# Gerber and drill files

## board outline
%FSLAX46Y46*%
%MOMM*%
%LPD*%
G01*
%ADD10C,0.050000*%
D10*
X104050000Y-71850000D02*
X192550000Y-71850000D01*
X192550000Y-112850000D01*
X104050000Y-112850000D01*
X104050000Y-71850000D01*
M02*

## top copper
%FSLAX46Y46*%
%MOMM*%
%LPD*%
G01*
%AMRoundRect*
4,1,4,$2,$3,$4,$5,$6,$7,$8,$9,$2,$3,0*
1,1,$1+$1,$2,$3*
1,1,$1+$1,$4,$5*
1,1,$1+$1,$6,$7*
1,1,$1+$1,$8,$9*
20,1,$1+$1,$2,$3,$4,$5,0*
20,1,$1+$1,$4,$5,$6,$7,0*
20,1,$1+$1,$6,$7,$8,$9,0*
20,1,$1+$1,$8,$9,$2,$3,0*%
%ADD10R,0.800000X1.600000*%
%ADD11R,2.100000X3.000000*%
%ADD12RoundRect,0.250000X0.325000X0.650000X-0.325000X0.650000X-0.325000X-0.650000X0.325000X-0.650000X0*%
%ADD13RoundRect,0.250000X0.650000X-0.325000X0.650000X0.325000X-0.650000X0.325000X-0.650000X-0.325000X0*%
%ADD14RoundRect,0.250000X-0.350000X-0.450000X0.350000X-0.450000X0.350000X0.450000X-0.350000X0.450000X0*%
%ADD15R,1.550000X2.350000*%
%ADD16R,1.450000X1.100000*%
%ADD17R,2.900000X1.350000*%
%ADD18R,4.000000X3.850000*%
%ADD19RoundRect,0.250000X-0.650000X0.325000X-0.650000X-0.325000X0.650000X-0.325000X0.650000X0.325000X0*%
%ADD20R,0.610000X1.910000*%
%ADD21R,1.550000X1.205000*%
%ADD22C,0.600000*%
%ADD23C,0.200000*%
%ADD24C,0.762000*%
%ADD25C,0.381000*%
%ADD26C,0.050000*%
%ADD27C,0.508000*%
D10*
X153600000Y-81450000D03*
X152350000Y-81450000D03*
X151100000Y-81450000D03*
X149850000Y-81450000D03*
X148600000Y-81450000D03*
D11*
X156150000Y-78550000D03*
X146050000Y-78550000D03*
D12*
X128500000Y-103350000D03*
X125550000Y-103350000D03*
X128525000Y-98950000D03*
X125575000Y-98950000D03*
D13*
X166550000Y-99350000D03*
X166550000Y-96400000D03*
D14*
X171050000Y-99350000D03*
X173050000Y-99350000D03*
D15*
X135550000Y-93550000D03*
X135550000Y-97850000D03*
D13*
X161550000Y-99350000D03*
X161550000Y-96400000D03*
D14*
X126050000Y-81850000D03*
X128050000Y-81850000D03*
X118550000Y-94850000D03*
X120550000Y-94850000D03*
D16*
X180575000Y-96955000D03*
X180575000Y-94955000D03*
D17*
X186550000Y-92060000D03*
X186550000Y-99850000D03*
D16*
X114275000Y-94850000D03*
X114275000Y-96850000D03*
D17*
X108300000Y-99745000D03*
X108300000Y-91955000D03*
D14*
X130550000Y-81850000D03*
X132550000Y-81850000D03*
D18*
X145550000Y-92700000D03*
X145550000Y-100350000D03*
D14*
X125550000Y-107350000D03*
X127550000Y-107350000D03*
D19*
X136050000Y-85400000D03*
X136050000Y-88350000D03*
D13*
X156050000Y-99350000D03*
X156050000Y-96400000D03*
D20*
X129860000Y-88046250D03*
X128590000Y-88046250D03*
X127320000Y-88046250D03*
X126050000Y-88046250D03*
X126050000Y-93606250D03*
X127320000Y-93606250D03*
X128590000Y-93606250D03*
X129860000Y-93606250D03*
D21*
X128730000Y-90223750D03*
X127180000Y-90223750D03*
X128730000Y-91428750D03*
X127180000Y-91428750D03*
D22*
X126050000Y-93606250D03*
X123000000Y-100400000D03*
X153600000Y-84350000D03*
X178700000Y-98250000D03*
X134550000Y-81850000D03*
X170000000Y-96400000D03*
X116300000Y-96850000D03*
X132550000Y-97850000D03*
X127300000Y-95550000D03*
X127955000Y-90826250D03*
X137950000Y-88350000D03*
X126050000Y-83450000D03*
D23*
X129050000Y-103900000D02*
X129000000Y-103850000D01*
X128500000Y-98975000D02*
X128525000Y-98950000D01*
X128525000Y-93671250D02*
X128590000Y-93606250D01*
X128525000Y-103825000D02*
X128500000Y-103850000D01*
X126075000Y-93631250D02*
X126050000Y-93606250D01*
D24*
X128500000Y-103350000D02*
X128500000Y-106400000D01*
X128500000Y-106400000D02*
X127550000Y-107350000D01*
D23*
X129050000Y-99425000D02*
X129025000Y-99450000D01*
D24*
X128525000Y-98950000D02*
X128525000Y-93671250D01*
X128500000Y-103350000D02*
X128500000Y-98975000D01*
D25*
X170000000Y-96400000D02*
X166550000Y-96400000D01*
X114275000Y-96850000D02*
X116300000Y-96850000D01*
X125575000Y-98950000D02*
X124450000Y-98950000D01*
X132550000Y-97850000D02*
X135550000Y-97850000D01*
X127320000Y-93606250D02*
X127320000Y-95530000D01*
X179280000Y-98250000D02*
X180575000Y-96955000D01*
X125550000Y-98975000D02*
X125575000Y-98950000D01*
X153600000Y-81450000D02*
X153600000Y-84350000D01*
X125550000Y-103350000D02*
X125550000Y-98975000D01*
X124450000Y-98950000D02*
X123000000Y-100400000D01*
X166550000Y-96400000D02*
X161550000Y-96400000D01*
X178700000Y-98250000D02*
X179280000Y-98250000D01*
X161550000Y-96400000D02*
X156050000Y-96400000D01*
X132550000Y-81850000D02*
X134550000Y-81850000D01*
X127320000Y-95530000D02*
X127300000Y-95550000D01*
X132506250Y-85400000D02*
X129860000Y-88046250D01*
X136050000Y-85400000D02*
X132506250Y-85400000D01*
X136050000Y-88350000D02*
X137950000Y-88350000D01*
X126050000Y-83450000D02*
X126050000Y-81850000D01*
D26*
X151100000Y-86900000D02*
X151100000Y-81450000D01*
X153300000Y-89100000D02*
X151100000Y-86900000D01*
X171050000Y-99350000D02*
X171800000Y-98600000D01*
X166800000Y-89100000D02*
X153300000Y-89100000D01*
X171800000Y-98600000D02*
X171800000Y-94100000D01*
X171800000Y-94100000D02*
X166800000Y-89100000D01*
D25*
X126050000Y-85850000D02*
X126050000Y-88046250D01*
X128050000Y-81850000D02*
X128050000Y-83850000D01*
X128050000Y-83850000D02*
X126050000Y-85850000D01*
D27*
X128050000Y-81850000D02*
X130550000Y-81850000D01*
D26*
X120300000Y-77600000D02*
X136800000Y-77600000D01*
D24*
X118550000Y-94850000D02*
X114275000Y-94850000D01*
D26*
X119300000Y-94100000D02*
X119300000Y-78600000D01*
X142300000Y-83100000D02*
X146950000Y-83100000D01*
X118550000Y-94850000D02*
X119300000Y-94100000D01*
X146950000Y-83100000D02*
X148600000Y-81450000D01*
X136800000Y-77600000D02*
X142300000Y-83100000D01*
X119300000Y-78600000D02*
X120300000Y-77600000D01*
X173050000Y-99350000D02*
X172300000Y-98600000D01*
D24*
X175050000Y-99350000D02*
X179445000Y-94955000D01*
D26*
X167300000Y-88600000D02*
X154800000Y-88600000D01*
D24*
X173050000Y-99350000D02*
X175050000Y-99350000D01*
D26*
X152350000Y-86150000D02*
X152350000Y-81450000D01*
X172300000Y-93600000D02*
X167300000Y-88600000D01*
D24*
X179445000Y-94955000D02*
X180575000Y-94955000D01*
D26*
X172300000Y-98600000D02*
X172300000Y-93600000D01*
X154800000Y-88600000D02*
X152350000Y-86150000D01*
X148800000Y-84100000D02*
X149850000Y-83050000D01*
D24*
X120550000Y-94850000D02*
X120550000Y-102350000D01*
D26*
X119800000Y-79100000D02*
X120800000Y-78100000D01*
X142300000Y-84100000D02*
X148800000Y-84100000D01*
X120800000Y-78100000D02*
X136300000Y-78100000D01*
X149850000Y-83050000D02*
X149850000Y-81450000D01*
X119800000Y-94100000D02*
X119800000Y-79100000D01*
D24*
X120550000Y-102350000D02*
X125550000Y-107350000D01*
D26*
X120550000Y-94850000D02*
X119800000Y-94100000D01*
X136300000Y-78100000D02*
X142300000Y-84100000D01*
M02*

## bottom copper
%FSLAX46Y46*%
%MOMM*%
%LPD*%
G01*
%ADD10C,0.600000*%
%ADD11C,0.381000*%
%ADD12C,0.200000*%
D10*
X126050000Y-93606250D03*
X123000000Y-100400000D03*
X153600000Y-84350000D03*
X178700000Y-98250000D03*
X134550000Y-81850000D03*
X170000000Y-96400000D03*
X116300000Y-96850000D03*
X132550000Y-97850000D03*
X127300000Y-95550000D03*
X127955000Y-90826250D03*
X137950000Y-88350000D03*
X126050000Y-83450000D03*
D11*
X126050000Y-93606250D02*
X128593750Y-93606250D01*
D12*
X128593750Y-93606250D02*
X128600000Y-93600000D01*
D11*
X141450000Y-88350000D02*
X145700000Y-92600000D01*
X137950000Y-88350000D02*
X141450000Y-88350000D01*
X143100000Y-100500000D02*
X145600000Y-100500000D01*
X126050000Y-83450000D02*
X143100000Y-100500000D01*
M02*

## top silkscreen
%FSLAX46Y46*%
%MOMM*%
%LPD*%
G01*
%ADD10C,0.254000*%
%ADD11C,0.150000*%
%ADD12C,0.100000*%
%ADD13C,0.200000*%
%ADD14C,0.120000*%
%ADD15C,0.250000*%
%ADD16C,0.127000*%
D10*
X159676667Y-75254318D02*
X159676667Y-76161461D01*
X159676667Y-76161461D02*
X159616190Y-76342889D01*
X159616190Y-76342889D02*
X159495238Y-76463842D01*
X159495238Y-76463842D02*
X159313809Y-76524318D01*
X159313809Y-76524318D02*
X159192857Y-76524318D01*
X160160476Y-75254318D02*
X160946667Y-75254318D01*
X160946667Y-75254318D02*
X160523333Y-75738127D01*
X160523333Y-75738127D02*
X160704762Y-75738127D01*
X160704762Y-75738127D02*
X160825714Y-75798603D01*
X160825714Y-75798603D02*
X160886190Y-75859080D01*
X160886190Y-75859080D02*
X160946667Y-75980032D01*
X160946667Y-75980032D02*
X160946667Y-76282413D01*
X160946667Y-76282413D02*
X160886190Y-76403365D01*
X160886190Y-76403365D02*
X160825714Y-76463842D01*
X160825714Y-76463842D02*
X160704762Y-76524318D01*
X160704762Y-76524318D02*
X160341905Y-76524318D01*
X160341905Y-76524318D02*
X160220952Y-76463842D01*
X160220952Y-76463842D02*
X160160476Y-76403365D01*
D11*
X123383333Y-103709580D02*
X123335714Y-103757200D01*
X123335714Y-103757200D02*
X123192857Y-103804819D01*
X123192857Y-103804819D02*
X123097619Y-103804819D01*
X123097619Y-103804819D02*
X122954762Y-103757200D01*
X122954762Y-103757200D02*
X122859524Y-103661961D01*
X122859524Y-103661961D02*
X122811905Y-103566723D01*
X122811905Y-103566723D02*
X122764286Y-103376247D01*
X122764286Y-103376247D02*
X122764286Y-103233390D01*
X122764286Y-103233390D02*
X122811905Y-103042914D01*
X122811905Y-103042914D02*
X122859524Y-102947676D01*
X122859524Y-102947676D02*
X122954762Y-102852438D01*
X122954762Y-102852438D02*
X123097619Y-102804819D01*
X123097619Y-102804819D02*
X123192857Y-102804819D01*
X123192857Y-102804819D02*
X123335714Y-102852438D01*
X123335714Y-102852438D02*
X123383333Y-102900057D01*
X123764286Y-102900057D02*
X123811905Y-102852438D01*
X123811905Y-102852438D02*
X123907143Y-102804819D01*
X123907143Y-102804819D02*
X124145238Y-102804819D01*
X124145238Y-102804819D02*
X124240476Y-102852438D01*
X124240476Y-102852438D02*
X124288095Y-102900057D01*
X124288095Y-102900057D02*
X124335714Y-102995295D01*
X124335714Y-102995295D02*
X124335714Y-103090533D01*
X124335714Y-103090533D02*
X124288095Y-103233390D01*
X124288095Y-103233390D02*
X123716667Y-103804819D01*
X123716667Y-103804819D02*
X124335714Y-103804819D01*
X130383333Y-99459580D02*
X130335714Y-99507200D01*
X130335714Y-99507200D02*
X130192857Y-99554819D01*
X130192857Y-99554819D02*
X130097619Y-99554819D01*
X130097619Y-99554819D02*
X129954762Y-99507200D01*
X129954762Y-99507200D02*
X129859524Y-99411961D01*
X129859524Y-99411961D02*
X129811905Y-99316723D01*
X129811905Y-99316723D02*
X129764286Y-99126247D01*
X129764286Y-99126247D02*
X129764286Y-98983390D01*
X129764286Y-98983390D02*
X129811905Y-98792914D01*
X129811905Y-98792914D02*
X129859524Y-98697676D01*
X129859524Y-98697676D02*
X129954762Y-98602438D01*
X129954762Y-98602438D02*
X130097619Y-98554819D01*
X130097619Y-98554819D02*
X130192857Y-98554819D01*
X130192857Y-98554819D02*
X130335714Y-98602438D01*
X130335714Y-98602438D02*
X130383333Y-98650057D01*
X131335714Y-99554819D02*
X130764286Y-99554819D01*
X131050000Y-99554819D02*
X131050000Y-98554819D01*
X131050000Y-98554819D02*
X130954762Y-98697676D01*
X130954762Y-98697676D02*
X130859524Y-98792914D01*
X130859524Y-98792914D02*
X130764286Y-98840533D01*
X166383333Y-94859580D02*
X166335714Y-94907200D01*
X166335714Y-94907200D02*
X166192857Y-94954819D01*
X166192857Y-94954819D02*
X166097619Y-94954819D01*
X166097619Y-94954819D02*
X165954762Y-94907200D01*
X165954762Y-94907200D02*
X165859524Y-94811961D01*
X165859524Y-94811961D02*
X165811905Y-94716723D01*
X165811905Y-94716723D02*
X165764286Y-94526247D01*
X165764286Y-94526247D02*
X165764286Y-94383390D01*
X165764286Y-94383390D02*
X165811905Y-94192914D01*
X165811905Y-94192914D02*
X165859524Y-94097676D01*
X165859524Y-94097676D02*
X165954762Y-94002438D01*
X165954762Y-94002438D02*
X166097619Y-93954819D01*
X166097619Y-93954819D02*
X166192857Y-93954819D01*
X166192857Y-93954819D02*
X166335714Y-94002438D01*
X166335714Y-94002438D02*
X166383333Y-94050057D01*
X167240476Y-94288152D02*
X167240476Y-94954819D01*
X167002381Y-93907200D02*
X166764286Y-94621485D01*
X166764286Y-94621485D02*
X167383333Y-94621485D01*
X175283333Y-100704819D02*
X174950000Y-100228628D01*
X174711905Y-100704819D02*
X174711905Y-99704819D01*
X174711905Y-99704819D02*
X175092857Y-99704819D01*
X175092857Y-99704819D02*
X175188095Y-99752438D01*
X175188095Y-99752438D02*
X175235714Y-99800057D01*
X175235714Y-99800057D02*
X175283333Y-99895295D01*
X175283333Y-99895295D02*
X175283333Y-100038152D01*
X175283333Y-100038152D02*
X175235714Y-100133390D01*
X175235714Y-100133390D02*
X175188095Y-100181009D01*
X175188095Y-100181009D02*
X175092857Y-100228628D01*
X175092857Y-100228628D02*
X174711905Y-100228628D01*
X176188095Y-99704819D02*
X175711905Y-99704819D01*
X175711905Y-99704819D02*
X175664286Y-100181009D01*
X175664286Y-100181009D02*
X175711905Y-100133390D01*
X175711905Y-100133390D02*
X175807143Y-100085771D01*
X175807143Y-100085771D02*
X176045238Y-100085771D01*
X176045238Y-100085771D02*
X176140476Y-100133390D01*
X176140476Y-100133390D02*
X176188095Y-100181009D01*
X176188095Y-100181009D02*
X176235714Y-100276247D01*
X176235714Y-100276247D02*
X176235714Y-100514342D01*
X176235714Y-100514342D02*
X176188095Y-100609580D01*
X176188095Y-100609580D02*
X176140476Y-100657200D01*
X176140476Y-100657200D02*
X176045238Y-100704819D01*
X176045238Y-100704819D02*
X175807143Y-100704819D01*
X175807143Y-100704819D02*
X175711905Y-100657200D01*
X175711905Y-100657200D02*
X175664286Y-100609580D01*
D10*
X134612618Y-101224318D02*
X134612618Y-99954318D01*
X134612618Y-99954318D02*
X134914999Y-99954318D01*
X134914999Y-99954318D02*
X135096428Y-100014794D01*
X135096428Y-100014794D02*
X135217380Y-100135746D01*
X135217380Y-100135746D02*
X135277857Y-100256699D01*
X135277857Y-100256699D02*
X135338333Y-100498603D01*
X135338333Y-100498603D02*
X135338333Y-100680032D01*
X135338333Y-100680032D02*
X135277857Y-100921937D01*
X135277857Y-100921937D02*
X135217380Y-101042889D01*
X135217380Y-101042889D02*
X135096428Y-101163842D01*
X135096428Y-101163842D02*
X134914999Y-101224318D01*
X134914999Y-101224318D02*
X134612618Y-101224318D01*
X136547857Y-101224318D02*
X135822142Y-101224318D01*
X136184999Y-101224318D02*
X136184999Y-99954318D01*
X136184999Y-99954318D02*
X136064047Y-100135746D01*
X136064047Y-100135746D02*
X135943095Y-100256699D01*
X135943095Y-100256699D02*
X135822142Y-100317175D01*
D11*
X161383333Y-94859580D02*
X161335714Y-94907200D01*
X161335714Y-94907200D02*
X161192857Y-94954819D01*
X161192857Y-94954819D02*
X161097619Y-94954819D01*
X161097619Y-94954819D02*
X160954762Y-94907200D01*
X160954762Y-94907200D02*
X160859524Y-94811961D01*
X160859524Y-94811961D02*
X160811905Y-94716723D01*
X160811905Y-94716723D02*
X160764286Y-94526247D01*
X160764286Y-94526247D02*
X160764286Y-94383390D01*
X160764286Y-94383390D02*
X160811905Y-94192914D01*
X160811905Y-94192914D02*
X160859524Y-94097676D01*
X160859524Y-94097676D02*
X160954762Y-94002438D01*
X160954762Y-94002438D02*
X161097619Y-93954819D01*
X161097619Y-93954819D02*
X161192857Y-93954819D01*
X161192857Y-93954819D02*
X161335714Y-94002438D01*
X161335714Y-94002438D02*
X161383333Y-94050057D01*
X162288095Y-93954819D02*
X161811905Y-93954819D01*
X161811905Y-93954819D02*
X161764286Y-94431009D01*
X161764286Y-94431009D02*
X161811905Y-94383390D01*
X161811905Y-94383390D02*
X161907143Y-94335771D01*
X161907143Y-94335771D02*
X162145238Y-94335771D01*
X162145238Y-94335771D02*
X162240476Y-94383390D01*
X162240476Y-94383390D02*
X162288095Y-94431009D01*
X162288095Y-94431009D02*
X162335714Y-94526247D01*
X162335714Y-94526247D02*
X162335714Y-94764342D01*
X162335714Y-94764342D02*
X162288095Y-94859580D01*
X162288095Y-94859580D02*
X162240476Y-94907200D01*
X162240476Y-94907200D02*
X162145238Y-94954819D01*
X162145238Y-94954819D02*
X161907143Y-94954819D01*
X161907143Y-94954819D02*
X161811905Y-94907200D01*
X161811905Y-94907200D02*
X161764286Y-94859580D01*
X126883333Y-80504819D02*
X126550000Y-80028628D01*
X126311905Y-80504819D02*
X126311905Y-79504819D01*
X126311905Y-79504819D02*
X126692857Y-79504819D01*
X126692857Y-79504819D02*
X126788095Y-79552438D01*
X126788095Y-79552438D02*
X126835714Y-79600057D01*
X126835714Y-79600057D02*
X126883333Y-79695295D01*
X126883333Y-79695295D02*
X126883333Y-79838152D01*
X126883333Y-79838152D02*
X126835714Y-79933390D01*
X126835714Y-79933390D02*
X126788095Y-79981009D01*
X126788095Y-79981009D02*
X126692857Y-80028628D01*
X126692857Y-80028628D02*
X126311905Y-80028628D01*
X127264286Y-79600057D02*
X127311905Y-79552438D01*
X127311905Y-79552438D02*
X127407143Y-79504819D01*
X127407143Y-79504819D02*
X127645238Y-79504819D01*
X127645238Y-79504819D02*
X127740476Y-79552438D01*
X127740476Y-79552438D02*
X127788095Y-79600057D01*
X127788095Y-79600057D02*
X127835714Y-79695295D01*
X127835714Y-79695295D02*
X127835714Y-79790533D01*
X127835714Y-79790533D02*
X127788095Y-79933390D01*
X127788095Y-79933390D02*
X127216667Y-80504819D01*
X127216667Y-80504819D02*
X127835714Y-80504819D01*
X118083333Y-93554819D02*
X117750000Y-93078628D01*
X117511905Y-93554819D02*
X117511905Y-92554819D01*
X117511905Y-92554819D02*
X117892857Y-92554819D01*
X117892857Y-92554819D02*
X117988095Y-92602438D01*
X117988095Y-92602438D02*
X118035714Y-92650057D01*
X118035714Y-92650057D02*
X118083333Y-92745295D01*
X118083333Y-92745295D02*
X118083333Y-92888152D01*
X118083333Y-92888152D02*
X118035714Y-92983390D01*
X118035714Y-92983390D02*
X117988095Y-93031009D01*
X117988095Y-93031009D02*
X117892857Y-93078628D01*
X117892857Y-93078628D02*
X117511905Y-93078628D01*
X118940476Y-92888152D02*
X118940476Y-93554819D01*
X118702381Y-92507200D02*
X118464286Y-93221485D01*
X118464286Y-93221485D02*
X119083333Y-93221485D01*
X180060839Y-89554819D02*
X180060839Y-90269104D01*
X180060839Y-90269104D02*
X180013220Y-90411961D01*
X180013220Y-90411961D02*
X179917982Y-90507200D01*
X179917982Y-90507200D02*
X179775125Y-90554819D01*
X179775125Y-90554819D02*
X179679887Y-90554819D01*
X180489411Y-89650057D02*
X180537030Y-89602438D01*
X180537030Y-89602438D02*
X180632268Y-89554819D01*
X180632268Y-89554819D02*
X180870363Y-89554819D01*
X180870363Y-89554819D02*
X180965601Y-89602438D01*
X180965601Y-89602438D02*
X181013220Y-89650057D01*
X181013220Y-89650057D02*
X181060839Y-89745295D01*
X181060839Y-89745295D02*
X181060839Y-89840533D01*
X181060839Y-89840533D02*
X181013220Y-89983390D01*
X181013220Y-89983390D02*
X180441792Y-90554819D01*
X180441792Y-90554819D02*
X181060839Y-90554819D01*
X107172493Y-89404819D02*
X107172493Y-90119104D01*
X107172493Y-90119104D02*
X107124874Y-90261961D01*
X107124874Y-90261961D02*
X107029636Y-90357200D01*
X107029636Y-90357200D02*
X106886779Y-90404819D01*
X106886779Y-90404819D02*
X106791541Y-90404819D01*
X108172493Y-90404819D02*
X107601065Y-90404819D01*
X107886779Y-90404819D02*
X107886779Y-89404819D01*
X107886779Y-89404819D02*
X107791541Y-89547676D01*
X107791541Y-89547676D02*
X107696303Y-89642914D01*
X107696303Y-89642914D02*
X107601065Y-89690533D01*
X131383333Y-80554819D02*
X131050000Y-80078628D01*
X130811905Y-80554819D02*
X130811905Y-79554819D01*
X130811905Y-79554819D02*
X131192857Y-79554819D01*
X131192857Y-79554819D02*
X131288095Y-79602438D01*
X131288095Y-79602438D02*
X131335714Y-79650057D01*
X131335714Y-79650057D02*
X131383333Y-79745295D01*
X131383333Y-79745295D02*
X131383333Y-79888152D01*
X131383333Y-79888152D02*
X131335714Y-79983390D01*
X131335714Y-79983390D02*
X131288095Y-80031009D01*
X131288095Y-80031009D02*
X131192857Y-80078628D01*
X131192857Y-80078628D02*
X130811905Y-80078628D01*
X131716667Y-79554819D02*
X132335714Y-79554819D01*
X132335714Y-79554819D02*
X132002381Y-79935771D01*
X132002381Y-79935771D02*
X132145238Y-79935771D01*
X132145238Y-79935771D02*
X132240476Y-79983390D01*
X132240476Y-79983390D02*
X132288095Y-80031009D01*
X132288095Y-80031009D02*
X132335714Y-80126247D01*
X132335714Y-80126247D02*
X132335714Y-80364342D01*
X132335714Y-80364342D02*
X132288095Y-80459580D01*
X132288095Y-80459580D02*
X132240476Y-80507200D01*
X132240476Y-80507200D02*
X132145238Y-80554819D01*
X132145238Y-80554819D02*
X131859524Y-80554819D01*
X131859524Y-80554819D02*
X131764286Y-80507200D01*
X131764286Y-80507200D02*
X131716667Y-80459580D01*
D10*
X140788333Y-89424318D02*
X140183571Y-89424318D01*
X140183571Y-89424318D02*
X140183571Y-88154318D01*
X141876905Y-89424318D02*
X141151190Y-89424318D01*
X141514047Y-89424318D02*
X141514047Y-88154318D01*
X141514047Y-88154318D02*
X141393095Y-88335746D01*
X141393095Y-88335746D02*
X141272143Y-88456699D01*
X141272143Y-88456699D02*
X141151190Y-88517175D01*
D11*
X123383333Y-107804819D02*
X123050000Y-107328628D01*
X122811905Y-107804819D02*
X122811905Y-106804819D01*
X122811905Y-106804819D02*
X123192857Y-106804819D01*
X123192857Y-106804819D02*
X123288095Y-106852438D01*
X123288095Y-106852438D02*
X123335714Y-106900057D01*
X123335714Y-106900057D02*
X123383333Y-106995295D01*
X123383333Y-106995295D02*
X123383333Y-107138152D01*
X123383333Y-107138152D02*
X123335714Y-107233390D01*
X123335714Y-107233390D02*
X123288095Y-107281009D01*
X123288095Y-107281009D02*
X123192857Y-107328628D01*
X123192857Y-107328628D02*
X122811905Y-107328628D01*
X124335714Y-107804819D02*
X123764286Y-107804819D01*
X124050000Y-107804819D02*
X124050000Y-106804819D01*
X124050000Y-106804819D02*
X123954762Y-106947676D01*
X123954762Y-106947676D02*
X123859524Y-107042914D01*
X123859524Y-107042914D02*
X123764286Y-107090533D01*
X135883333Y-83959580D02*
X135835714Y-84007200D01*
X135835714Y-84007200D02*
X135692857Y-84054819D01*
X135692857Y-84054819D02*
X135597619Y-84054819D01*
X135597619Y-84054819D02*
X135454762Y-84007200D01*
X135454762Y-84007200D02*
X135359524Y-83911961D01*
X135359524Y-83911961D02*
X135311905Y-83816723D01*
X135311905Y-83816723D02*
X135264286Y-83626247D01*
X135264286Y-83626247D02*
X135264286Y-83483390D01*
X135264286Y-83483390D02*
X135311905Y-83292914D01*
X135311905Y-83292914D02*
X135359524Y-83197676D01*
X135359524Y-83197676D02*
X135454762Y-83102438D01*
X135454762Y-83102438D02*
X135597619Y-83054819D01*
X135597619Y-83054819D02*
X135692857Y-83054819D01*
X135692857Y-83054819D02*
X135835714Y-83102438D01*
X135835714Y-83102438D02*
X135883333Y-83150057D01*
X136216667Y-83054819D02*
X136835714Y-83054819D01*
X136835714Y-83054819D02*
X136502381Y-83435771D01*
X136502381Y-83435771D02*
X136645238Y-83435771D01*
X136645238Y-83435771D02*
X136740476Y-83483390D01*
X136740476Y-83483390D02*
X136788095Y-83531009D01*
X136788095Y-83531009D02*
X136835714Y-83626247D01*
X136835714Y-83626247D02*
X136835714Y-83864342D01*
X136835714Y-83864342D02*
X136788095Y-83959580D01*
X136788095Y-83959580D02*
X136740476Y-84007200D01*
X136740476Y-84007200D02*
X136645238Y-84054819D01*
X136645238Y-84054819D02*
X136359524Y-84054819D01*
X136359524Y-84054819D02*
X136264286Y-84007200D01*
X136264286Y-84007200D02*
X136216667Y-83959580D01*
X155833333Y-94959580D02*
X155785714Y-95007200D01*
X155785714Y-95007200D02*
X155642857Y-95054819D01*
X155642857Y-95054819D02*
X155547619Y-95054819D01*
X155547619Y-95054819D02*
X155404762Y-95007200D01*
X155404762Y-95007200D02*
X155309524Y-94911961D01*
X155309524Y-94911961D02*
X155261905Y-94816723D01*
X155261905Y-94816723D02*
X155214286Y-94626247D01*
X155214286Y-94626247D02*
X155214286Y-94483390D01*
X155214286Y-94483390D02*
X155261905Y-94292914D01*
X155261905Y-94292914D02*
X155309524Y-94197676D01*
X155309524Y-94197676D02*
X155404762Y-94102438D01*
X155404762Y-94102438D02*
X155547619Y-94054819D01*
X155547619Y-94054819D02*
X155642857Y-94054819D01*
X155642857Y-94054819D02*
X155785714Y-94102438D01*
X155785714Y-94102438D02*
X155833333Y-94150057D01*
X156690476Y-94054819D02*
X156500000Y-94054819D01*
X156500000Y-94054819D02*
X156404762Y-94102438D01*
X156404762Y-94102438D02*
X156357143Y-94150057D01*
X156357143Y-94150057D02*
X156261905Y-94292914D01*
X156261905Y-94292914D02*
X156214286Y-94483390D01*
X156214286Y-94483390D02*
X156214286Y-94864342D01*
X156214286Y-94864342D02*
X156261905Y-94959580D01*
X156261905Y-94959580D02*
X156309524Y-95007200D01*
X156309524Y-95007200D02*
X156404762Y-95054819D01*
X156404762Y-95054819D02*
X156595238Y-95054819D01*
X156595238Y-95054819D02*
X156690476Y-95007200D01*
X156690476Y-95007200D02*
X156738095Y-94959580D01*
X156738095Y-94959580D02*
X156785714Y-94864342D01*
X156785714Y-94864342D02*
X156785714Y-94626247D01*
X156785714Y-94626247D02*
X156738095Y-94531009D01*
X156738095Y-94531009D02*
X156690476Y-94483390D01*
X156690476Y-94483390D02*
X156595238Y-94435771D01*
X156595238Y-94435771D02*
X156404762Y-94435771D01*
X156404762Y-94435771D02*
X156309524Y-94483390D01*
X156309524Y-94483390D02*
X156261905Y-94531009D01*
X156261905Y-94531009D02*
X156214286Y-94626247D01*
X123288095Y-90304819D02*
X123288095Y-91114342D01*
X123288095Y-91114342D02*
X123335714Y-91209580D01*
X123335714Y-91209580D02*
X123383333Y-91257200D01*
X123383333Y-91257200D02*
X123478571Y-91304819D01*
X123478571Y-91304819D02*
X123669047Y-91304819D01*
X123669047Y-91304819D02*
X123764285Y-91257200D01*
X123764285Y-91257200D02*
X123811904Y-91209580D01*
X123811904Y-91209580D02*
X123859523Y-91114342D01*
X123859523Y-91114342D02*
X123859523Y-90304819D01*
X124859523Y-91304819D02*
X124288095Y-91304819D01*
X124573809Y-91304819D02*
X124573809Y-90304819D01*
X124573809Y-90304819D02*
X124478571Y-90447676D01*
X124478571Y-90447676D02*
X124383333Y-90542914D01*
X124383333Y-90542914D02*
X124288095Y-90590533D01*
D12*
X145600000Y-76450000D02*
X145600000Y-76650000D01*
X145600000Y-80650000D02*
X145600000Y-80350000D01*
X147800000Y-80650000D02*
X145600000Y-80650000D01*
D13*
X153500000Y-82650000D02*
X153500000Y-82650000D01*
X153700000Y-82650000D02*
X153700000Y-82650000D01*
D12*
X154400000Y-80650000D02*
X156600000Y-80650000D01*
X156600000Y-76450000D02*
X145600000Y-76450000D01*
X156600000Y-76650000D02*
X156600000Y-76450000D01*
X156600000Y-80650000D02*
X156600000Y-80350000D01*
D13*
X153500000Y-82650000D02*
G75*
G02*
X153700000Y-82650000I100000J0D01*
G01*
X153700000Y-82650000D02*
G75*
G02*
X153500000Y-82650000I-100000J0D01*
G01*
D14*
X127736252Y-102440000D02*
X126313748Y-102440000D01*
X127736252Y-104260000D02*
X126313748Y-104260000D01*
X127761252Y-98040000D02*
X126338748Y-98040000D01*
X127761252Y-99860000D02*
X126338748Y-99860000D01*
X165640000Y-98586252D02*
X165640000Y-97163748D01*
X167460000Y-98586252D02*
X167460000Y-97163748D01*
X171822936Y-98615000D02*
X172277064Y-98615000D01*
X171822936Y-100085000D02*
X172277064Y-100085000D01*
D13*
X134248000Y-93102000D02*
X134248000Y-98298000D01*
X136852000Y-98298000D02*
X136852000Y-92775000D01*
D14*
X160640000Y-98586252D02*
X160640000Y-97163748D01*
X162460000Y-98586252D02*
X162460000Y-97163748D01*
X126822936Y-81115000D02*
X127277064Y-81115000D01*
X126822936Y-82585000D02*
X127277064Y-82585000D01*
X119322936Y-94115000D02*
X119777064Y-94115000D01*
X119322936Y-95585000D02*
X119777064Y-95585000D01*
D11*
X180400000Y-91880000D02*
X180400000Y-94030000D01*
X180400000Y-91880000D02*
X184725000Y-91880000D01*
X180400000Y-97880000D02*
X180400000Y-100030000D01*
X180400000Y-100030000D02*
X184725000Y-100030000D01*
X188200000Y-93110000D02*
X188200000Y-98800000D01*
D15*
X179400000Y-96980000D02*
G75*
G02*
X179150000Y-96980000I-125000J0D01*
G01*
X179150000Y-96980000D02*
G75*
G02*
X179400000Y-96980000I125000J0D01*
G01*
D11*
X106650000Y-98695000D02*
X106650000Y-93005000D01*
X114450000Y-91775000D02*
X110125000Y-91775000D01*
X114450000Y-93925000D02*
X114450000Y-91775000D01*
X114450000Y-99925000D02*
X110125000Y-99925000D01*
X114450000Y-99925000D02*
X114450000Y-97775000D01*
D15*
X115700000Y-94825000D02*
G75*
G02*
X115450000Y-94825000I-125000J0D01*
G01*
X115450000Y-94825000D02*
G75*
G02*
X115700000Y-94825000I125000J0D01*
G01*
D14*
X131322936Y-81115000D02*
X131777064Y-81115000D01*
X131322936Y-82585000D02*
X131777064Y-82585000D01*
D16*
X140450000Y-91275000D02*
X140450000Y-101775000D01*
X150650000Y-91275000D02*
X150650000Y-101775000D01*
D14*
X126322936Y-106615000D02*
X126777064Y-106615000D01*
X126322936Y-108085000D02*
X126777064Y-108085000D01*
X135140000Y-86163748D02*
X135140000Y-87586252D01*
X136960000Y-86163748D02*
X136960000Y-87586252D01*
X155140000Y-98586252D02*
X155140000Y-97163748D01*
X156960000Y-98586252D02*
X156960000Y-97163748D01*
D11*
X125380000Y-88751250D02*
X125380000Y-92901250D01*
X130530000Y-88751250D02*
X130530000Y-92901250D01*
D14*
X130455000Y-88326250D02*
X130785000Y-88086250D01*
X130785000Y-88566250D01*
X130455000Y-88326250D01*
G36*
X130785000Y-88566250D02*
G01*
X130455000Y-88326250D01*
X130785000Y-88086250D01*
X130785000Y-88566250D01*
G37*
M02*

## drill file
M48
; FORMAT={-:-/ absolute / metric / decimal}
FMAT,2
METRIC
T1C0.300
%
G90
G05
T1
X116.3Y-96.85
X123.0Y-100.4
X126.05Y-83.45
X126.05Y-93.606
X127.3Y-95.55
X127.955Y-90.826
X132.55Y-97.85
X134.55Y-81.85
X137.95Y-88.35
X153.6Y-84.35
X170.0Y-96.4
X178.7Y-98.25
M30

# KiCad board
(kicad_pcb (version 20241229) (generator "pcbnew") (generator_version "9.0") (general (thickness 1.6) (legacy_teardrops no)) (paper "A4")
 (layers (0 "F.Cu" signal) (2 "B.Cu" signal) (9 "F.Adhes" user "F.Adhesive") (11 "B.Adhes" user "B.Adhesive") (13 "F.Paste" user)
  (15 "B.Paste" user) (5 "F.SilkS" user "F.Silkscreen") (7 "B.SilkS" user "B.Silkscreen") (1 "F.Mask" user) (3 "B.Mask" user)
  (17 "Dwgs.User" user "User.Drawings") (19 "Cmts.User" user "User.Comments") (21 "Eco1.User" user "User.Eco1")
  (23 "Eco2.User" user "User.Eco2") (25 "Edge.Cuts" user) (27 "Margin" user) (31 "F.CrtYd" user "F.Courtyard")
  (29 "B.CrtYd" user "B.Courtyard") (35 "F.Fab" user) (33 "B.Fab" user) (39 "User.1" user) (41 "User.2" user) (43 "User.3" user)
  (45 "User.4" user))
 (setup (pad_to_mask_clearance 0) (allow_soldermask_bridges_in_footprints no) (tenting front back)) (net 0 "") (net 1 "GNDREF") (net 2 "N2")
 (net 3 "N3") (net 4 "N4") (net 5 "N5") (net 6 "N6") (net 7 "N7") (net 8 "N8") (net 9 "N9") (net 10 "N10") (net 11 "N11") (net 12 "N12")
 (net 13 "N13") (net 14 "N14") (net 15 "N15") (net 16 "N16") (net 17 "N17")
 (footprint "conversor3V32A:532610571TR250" (layer "F.Cu") (at 151.1 80.65 180)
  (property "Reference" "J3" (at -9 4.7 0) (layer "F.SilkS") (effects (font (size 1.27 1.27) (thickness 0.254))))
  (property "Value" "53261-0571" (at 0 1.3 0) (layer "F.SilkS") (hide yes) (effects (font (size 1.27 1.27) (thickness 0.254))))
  (fp_line (start 5.5 4.2) (end 5.5 4) (stroke (width 0.1) (type solid)) (layer "F.SilkS"))
  (fp_line (start 5.5 0) (end 5.5 0.3) (stroke (width 0.1) (type solid)) (layer "F.SilkS"))
  (fp_line (start 3.3 0) (end 5.5 0) (stroke (width 0.1) (type solid)) (layer "F.SilkS"))
  (fp_line (start -2.4 -2) (end -2.4 -2) (stroke (width 0.2) (type solid)) (layer "F.SilkS"))
  (fp_line (start -2.6 -2) (end -2.6 -2) (stroke (width 0.2) (type solid)) (layer "F.SilkS"))
  (fp_line (start -3.3 0) (end -5.5 0) (stroke (width 0.1) (type solid)) (layer "F.SilkS"))
  (fp_line (start -5.5 4.2) (end 5.5 4.2) (stroke (width 0.1) (type solid)) (layer "F.SilkS"))
  (fp_line (start -5.5 4) (end -5.5 4.2) (stroke (width 0.1) (type solid)) (layer "F.SilkS"))
  (fp_line (start -5.5 0) (end -5.5 0.3) (stroke (width 0.1) (type solid)) (layer "F.SilkS"))
  (fp_arc (start -2.4 -2) (mid -2.5 -1.9) (end -2.6 -2) (stroke (width 0.2) (type solid)) (layer "F.SilkS"))
  (fp_arc (start -2.6 -2) (mid -2.5 -2.1) (end -2.4 -2) (stroke (width 0.2) (type solid)) (layer "F.SilkS"))
  (pad "1" smd rect (at -2.5 -0.8 180) (size 0.8 1.6) (layers "F.Cu" "F.Mask" "F.Paste") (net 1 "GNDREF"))
  (pad "2" smd rect (at -1.25 -0.8 180) (size 0.8 1.6) (layers "F.Cu" "F.Mask" "F.Paste") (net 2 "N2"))
  (pad "3" smd rect (at 0 -0.8 180) (size 0.8 1.6) (layers "F.Cu" "F.Mask" "F.Paste") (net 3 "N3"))
  (pad "4" smd rect (at 1.25 -0.8 180) (size 0.8 1.6) (layers "F.Cu" "F.Mask" "F.Paste") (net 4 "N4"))
  (pad "5" smd rect (at 2.5 -0.8 180) (size 0.8 1.6) (layers "F.Cu" "F.Mask" "F.Paste") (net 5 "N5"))
  (pad "MP1" smd rect (at -5.05 2.1 180) (size 2.1 3) (layers "F.Cu" "F.Mask" "F.Paste") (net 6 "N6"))
  (pad "MP2" smd rect (at 5.05 2.1 180) (size 2.1 3) (layers "F.Cu" "F.Mask" "F.Paste") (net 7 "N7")))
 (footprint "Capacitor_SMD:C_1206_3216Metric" (layer "F.Cu") (at 127.025 103.35 180)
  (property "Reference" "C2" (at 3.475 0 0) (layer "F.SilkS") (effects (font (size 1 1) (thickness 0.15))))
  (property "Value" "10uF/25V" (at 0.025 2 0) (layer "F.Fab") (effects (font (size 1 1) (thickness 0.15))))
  (fp_line (start -0.711252 0.91) (end 0.711252 0.91) (stroke (width 0.12) (type solid)) (layer "F.SilkS"))
  (fp_line (start -0.711252 -0.91) (end 0.711252 -0.91) (stroke (width 0.12) (type solid)) (layer "F.SilkS"))
  (pad "1" smd roundrect (at -1.475 0 180) (size 1.15 1.8) (layers "F.Cu" "F.Mask" "F.Paste") (roundrect_rratio 0.217391) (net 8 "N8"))
  (pad "2" smd roundrect (at 1.475 0 180) (size 1.15 1.8) (layers "F.Cu" "F.Mask" "F.Paste") (roundrect_rratio 0.217391) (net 1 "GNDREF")))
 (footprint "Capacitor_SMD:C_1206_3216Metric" (layer "F.Cu") (at 127.05 98.95 180)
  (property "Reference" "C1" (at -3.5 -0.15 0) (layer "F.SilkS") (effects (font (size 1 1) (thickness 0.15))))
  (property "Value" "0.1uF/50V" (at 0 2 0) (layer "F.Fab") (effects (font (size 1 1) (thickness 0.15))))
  (fp_line (start -0.711252 0.91) (end 0.711252 0.91) (stroke (width 0.12) (type solid)) (layer "F.SilkS"))
  (fp_line (start -0.711252 -0.91) (end 0.711252 -0.91) (stroke (width 0.12) (type solid)) (layer "F.SilkS"))
  (pad "1" smd roundrect (at -1.475 0 180) (size 1.15 1.8) (layers "F.Cu" "F.Mask" "F.Paste") (roundrect_rratio 0.217391) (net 8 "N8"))
  (pad "2" smd roundrect (at 1.475 0 180) (size 1.15 1.8) (layers "F.Cu" "F.Mask" "F.Paste") (roundrect_rratio 0.217391) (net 1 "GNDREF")))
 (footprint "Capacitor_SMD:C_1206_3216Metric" (layer "F.Cu") (at 166.55 97.875 90)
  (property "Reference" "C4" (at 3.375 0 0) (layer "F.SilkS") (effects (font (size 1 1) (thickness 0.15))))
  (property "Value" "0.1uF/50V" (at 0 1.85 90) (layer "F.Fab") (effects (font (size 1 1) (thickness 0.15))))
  (fp_line (start -0.711252 -0.91) (end 0.711252 -0.91) (stroke (width 0.12) (type solid)) (layer "F.SilkS"))
  (fp_line (start -0.711252 0.91) (end 0.711252 0.91) (stroke (width 0.12) (type solid)) (layer "F.SilkS"))
  (pad "1" smd roundrect (at -1.475 0 90) (size 1.15 1.8) (layers "F.Cu" "F.Mask" "F.Paste") (roundrect_rratio 0.217391) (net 3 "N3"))
  (pad "2" smd roundrect (at 1.475 0 90) (size 1.15 1.8) (layers "F.Cu" "F.Mask" "F.Paste") (roundrect_rratio 0.217391) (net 1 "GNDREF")))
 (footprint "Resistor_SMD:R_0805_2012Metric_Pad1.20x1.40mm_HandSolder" (layer "F.Cu") (at 172.05 99.35)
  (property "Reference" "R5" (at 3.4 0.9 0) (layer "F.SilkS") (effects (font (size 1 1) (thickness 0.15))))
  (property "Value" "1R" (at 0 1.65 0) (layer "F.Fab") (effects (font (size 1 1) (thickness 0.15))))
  (fp_line (start -0.227064 -0.735) (end 0.227064 -0.735) (stroke (width 0.12) (type solid)) (layer "F.SilkS"))
  (fp_line (start -0.227064 0.735) (end 0.227064 0.735) (stroke (width 0.12) (type solid)) (layer "F.SilkS"))
  (pad "1" smd roundrect (at -1 0) (size 1.2 1.4) (layers "F.Cu" "F.Mask" "F.Paste") (roundrect_rratio 0.208333) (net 3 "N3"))
  (pad "2" smd roundrect (at 1 0) (size 1.2 1.4) (layers "F.Cu" "F.Mask" "F.Paste") (roundrect_rratio 0.208333) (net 2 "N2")))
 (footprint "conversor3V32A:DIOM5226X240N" (layer "F.Cu") (at 135.55 95.7 -90)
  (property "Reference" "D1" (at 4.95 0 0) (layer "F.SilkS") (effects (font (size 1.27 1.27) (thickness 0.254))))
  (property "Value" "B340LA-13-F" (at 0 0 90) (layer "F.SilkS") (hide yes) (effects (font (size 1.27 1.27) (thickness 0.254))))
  (fp_line (start -2.598 1.302) (end 2.598 1.302) (stroke (width 0.2) (type solid)) (layer "F.SilkS"))
  (fp_line (start 2.598 -1.302) (end -2.925 -1.302) (stroke (width 0.2) (type solid)) (layer "F.SilkS"))
  (pad "1" smd rect (at -2.15 0) (size 1.55 2.35) (layers "F.Cu" "F.Mask" "F.Paste") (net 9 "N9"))
  (pad "2" smd rect (at 2.15 0) (size 1.55 2.35) (layers "F.Cu" "F.Mask" "F.Paste") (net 1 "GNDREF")))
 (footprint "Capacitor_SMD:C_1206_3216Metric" (layer "F.Cu") (at 161.55 97.875 90)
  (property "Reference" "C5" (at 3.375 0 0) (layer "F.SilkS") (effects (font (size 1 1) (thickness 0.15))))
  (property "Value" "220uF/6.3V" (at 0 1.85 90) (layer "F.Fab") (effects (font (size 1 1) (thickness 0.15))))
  (fp_line (start -0.711252 -0.91) (end 0.711252 -0.91) (stroke (width 0.12) (type solid)) (layer "F.SilkS"))
  (fp_line (start -0.711252 0.91) (end 0.711252 0.91) (stroke (width 0.12) (type solid)) (layer "F.SilkS"))
  (pad "1" smd roundrect (at -1.475 0 90) (size 1.15 1.8) (layers "F.Cu" "F.Mask" "F.Paste") (roundrect_rratio 0.217391) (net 3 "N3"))
  (pad "2" smd roundrect (at 1.475 0 90) (size 1.15 1.8) (layers "F.Cu" "F.Mask" "F.Paste") (roundrect_rratio 0.217391) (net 1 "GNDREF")))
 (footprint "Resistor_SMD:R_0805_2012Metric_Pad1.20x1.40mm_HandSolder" (layer "F.Cu") (at 127.05 81.85)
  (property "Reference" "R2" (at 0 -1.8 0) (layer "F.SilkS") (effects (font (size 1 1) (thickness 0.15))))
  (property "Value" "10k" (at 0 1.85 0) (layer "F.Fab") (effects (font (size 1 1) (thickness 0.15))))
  (fp_line (start -0.227064 -0.735) (end 0.227064 -0.735) (stroke (width 0.12) (type solid)) (layer "F.SilkS"))
  (fp_line (start -0.227064 0.735) (end 0.227064 0.735) (stroke (width 0.12) (type solid)) (layer "F.SilkS"))
  (pad "1" smd roundrect (at -1 0) (size 1.2 1.4) (layers "F.Cu" "F.Mask" "F.Paste") (roundrect_rratio 0.208333) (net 3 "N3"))
  (pad "2" smd roundrect (at 1 0) (size 1.2 1.4) (layers "F.Cu" "F.Mask" "F.Paste") (roundrect_rratio 0.208333) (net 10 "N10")))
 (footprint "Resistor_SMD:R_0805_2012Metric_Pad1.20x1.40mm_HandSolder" (layer "F.Cu") (at 119.55 94.85)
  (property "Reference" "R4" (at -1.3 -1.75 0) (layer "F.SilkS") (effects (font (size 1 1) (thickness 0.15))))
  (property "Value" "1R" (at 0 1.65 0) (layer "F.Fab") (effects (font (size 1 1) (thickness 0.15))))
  (fp_line (start -0.227064 -0.735) (end 0.227064 -0.735) (stroke (width 0.12) (type solid)) (layer "F.SilkS"))
  (fp_line (start -0.227064 0.735) (end 0.227064 0.735) (stroke (width 0.12) (type solid)) (layer "F.SilkS"))
  (pad "1" smd roundrect (at -1 0) (size 1.2 1.4) (layers "F.Cu" "F.Mask" "F.Paste") (roundrect_rratio 0.208333) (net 5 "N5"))
  (pad "2" smd roundrect (at 1 0) (size 1.2 1.4) (layers "F.Cu" "F.Mask" "F.Paste") (roundrect_rratio 0.208333) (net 4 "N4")))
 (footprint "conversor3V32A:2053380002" (layer "F.Cu") (at 184.3 95.955 -90)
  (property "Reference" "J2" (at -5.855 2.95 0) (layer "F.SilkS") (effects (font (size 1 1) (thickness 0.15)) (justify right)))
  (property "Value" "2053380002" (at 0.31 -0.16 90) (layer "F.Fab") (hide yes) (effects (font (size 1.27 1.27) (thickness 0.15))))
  (fp_line (start -4.075 3.9) (end -1.925 3.9) (stroke (width 0.15) (type solid)) (layer "F.SilkS"))
  (fp_line (start -4.075 3.9) (end -4.075 -0.425) (stroke (width 0.15) (type solid)) (layer "F.SilkS"))
  (fp_line (start 1.925 3.9) (end 4.075 3.9) (stroke (width 0.15) (type solid)) (layer "F.SilkS"))
  (fp_line (start 4.075 3.9) (end 4.075 -0.425) (stroke (width 0.15) (type solid)) (layer "F.SilkS"))
  (fp_line (start -2.845 -3.9) (end 2.845 -3.9) (stroke (width 0.15) (type solid)) (layer "F.SilkS"))
  (fp_circle (center 1.025 5.025) (end 1.15 5.025) (stroke (width 0.25) (type solid)) (fill no) (layer "F.SilkS"))
  (pad "1" smd rect (at 1 3.725 270) (size 1.1 1.45) (layers "F.Cu" "F.Mask" "F.Paste") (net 1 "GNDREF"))
  (pad "2" smd rect (at -1 3.725 270) (size 1.1 1.45) (layers "F.Cu" "F.Mask" "F.Paste") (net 2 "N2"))
  (pad "3" smd rect (at -3.895 -2.25 270) (size 1.35 2.9) (layers "F.Cu" "F.Mask" "F.Paste") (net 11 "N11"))
  (pad "4" smd rect (at 3.895 -2.25 270) (size 1.35 2.9) (layers "F.Cu" "F.Mask" "F.Paste") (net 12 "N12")))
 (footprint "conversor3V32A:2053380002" (layer "F.Cu") (at 110.55 95.85 90)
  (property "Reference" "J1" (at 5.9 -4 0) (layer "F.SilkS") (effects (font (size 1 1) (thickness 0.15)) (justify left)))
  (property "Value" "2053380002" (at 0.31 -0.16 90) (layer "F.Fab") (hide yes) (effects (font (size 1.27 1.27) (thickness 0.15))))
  (fp_line (start -2.845 -3.9) (end 2.845 -3.9) (stroke (width 0.15) (type solid)) (layer "F.SilkS"))
  (fp_line (start 4.075 3.9) (end 4.075 -0.425) (stroke (width 0.15) (type solid)) (layer "F.SilkS"))
  (fp_line (start 1.925 3.9) (end 4.075 3.9) (stroke (width 0.15) (type solid)) (layer "F.SilkS"))
  (fp_line (start -4.075 3.9) (end -4.075 -0.425) (stroke (width 0.15) (type solid)) (layer "F.SilkS"))
  (fp_line (start -4.075 3.9) (end -1.925 3.9) (stroke (width 0.15) (type solid)) (layer "F.SilkS"))
  (fp_circle (center 1.025 5.025) (end 1.15 5.025) (stroke (width 0.25) (type solid)) (fill no) (layer "F.SilkS"))
  (pad "1" smd rect (at 1 3.725 90) (size 1.1 1.45) (layers "F.Cu" "F.Mask" "F.Paste") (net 5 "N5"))
  (pad "2" smd rect (at -1 3.725 90) (size 1.1 1.45) (layers "F.Cu" "F.Mask" "F.Paste") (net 1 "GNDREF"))
  (pad "3" smd rect (at -3.895 -2.25 90) (size 1.35 2.9) (layers "F.Cu" "F.Mask" "F.Paste") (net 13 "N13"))
  (pad "4" smd rect (at 3.895 -2.25 90) (size 1.35 2.9) (layers "F.Cu" "F.Mask" "F.Paste") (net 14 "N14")))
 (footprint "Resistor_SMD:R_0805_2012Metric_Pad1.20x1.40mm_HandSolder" (layer "F.Cu") (at 131.55 81.85)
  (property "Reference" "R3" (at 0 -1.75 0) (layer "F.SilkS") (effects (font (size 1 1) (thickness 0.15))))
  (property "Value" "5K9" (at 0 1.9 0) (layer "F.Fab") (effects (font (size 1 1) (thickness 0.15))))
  (fp_line (start -0.227064 -0.735) (end 0.227064 -0.735) (stroke (width 0.12) (type solid)) (layer "F.SilkS"))
  (fp_line (start -0.227064 0.735) (end 0.227064 0.735) (stroke (width 0.12) (type solid)) (layer "F.SilkS"))
  (pad "1" smd roundrect (at -1 0) (size 1.2 1.4) (layers "F.Cu" "F.Mask" "F.Paste") (roundrect_rratio 0.208333) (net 10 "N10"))
  (pad "2" smd roundrect (at 1 0) (size 1.2 1.4) (layers "F.Cu" "F.Mask" "F.Paste") (roundrect_rratio 0.208333) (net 1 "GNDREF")))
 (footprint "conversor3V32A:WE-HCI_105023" (layer "F.Cu") (at 145.55 96.525 -90)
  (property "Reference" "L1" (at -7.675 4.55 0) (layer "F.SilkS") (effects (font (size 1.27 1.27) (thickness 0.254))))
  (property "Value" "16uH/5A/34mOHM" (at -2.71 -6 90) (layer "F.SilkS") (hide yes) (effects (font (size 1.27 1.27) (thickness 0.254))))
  (fp_line (start -5.25 5.1) (end 5.25 5.1) (stroke (width 0.127) (type solid)) (layer "F.SilkS"))
  (fp_line (start -5.25 -5.1) (end 5.25 -5.1) (stroke (width 0.127) (type solid)) (layer "F.SilkS"))
  (pad "1" smd rect (at -3.825 0 270) (size 3.85 4) (layers "F.Cu" "F.Mask" "F.Paste") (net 9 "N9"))
  (pad "2" smd rect (at 3.825 0 270) (size 3.85 4) (layers "F.Cu" "F.Mask" "F.Paste") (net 3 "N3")))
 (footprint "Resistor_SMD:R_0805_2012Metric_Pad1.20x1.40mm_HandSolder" (layer "F.Cu") (at 126.55 107.35)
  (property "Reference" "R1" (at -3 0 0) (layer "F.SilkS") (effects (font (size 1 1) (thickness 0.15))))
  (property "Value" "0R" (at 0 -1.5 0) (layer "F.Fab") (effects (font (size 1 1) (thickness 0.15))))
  (fp_line (start -0.227064 -0.735) (end 0.227064 -0.735) (stroke (width 0.12) (type solid)) (layer "F.SilkS"))
  (fp_line (start -0.227064 0.735) (end 0.227064 0.735) (stroke (width 0.12) (type solid)) (layer "F.SilkS"))
  (pad "1" smd roundrect (at -1 0) (size 1.2 1.4) (layers "F.Cu" "F.Mask" "F.Paste") (roundrect_rratio 0.208333) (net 4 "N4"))
  (pad "2" smd roundrect (at 1 0) (size 1.2 1.4) (layers "F.Cu" "F.Mask" "F.Paste") (roundrect_rratio 0.208333) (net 8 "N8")))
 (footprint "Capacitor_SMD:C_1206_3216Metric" (layer "F.Cu") (at 136.05 86.875 -90)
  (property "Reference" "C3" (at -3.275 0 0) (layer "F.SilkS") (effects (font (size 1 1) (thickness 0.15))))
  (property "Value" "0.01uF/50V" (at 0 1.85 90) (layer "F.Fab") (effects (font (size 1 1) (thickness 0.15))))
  (fp_line (start -0.711252 0.91) (end 0.711252 0.91) (stroke (width 0.12) (type solid)) (layer "F.SilkS"))
  (fp_line (start -0.711252 -0.91) (end 0.711252 -0.91) (stroke (width 0.12) (type solid)) (layer "F.SilkS"))
  (pad "1" smd roundrect (at -1.475 0 270) (size 1.15 1.8) (layers "F.Cu" "F.Mask" "F.Paste") (roundrect_rratio 0.217391) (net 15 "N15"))
  (pad "2" smd roundrect (at 1.475 0 270) (size 1.15 1.8) (layers "F.Cu" "F.Mask" "F.Paste") (roundrect_rratio 0.217391) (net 9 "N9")))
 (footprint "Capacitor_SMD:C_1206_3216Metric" (layer "F.Cu") (at 156.05 97.875 90)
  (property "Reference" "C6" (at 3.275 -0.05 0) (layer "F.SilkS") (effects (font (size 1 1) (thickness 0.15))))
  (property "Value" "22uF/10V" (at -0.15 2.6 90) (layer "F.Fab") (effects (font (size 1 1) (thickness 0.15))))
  (fp_line (start -0.711252 -0.91) (end 0.711252 -0.91) (stroke (width 0.12) (type solid)) (layer "F.SilkS"))
  (fp_line (start -0.711252 0.91) (end 0.711252 0.91) (stroke (width 0.12) (type solid)) (layer "F.SilkS"))
  (pad "1" smd roundrect (at -1.475 0 90) (size 1.15 1.8) (layers "F.Cu" "F.Mask" "F.Paste") (roundrect_rratio 0.217391) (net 3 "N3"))
  (pad "2" smd roundrect (at 1.475 0 90) (size 1.15 1.8) (layers "F.Cu" "F.Mask" "F.Paste") (roundrect_rratio 0.217391) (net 1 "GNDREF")))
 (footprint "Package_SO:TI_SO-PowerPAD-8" (layer "F.Cu") (at 127.955 90.82625 -90)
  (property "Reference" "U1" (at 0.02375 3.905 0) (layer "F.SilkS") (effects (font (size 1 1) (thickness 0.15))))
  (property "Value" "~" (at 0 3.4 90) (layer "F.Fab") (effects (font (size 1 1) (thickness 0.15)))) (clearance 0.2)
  (fp_line (start -2.075 2.575) (end 2.075 2.575) (stroke (width 0.15) (type solid)) (layer "F.SilkS"))
  (fp_line (start -2.075 -2.575) (end 2.075 -2.575) (stroke (width 0.15) (type solid)) (layer "F.SilkS"))
  (fp_poly
   (pts (xy -2.5 -2.5) (xy -2.74 -2.83) (xy -2.26 -2.83) (xy -2.5 -2.5)) (stroke (width 0.12) (type solid)) (fill yes) (layer "F.SilkS"))
  (pad "1" smd rect (at -2.78 -1.905 270) (size 1.91 0.61) (layers "F.Cu" "F.Mask" "F.Paste") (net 15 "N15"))
  (pad "2" smd rect (at -2.78 -0.635 270) (size 1.91 0.61) (layers "F.Cu" "F.Mask" "F.Paste") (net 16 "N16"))
  (pad "3" smd rect (at -2.78 0.635 270) (size 1.91 0.61) (layers "F.Cu" "F.Mask" "F.Paste") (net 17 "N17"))
  (pad "4" smd rect (at -2.78 1.905 270) (size 1.91 0.61) (layers "F.Cu" "F.Mask" "F.Paste") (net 10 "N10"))
  (pad "5" smd rect (at 2.78 1.905 270) (size 1.91 0.61) (layers "F.Cu" "F.Mask" "F.Paste") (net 8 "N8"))
  (pad "6" smd rect (at 2.78 0.635 270) (size 1.91 0.61) (layers "F.Cu" "F.Mask" "F.Paste") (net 1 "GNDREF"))
  (pad "7" smd rect (at 2.78 -0.635 270) (size 1.91 0.61) (layers "F.Cu" "F.Mask" "F.Paste") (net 8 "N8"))
  (pad "8" smd rect (at 2.78 -1.905 270) (size 1.91 0.61) (layers "F.Cu" "F.Mask" "F.Paste") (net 9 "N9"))
  (pad "9" smd rect (at -0.6025 -0.775 270) (size 1.205 1.55) (layers "F.Cu" "F.Mask" "F.Paste") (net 1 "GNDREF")
   (solder_paste_margin_ratio -0.2))
  (pad "9" smd rect (at -0.6025 0.775 270) (size 1.205 1.55) (layers "F.Cu" "F.Mask" "F.Paste") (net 1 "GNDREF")
   (solder_paste_margin_ratio -0.2))
  (pad "9" smd rect (at 0.6025 -0.775 270) (size 1.205 1.55) (layers "F.Cu" "F.Mask" "F.Paste") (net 1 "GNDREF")
   (solder_paste_margin_ratio -0.2))
  (pad "9" smd rect (at 0.6025 0.775 270) (size 1.205 1.55) (layers "F.Cu" "F.Mask" "F.Paste") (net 1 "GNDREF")
   (solder_paste_margin_ratio -0.2)))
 (gr_rect (start 104.05 71.85) (end 192.55 112.85) (stroke (width 0.05) (type solid)) (fill no) (layer "Edge.Cuts"))
 (segment (start 129.05 103.9) (end 129 103.85) (width 0.2) (layer "F.Cu") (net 8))
 (segment (start 128.5 98.975) (end 128.525 98.95) (width 0.2) (layer "F.Cu") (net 8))
 (segment (start 128.525 93.67125) (end 128.59 93.60625) (width 0.2) (layer "F.Cu") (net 8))
 (segment (start 128.525 103.825) (end 128.5 103.85) (width 0.2) (layer "F.Cu") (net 8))
 (segment (start 126.075 93.63125) (end 126.05 93.60625) (width 0.2) (layer "F.Cu") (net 8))
 (segment (start 128.5 103.35) (end 128.5 106.4) (width 0.762) (layer "F.Cu") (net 8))
 (segment (start 128.5 106.4) (end 127.55 107.35) (width 0.762) (layer "F.Cu") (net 8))
 (segment (start 129.05 99.425) (end 129.025 99.45) (width 0.2) (layer "F.Cu") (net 8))
 (segment (start 128.525 98.95) (end 128.525 93.67125) (width 0.762) (layer "F.Cu") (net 8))
 (segment (start 128.5 103.35) (end 128.5 98.975) (width 0.762) (layer "F.Cu") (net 8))
 (via (at 126.05 93.60625) (size 0.6) (drill 0.3) (layers "F.Cu" "B.Cu") (free yes) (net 8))
 (segment (start 126.05 93.60625) (end 128.59375 93.60625) (width 0.381) (layer "B.Cu") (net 8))
 (segment (start 128.59375 93.60625) (end 128.6 93.6) (width 0.2) (layer "B.Cu") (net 8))
 (segment (start 170 96.4) (end 166.55 96.4) (width 0.381) (layer "F.Cu") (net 1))
 (segment (start 114.275 96.85) (end 116.3 96.85) (width 0.381) (layer "F.Cu") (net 1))
 (segment (start 125.575 98.95) (end 124.45 98.95) (width 0.381) (layer "F.Cu") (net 1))
 (segment (start 132.55 97.85) (end 135.55 97.85) (width 0.381) (layer "F.Cu") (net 1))
 (segment (start 127.32 93.60625) (end 127.32 95.53) (width 0.381) (layer "F.Cu") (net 1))
 (segment (start 179.28 98.25) (end 180.575 96.955) (width 0.381) (layer "F.Cu") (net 1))
 (segment (start 125.55 98.975) (end 125.575 98.95) (width 0.381) (layer "F.Cu") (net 1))
 (segment (start 153.6 81.45) (end 153.6 84.35) (width 0.381) (layer "F.Cu") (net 1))
 (segment (start 125.55 103.35) (end 125.55 98.975) (width 0.381) (layer "F.Cu") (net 1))
 (segment (start 124.45 98.95) (end 123 100.4) (width 0.381) (layer "F.Cu") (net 1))
 (segment (start 166.55 96.4) (end 161.55 96.4) (width 0.381) (layer "F.Cu") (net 1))
 (segment (start 178.7 98.25) (end 179.28 98.25) (width 0.381) (layer "F.Cu") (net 1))
 (segment (start 161.55 96.4) (end 156.05 96.4) (width 0.381) (layer "F.Cu") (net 1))
 (segment (start 132.55 81.85) (end 134.55 81.85) (width 0.381) (layer "F.Cu") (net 1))
 (segment (start 127.32 95.53) (end 127.3 95.55) (width 0.381) (layer "F.Cu") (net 1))
 (via (at 123 100.4) (size 0.6) (drill 0.3) (layers "F.Cu" "B.Cu") (free yes) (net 1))
 (via (at 153.6 84.35) (size 0.6) (drill 0.3) (layers "F.Cu" "B.Cu") (free yes) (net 1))
 (via (at 178.7 98.25) (size 0.6) (drill 0.3) (layers "F.Cu" "B.Cu") (free yes) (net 1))
 (via (at 134.55 81.85) (size 0.6) (drill 0.3) (layers "F.Cu" "B.Cu") (free yes) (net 1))
 (via (at 170 96.4) (size 0.6) (drill 0.3) (layers "F.Cu" "B.Cu") (free yes) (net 1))
 (via (at 116.3 96.85) (size 0.6) (drill 0.3) (layers "F.Cu" "B.Cu") (free yes) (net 1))
 (via (at 132.55 97.85) (size 0.6) (drill 0.3) (layers "F.Cu" "B.Cu") (free yes) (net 1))
 (via (at 127.3 95.55) (size 0.6) (drill 0.3) (layers "F.Cu" "B.Cu") (free yes) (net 1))
 (via (at 127.955 90.82625) (size 0.6) (drill 0.3) (layers "F.Cu" "B.Cu") (free yes) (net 1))
 (segment (start 132.50625 85.4) (end 129.86 88.04625) (width 0.381) (layer "F.Cu") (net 15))
 (segment (start 136.05 85.4) (end 132.50625 85.4) (width 0.381) (layer "F.Cu") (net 15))
 (segment (start 136.05 88.35) (end 137.95 88.35) (width 0.381) (layer "F.Cu") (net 9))
 (via (at 137.95 88.35) (size 0.6) (drill 0.3) (layers "F.Cu" "B.Cu") (free yes) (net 9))
 (segment (start 141.45 88.35) (end 145.7 92.6) (width 0.381) (layer "B.Cu") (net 9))
 (segment (start 137.95 88.35) (end 141.45 88.35) (width 0.381) (layer "B.Cu") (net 9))
 (segment (start 126.05 83.45) (end 126.05 81.85) (width 0.381) (layer "F.Cu") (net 3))
 (segment (start 151.1 86.9) (end 151.1 81.45) (width 0.05) (layer "F.Cu") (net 3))
 (segment (start 153.3 89.1) (end 151.1 86.9) (width 0.05) (layer "F.Cu") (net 3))
 (segment (start 171.05 99.35) (end 171.8 98.6) (width 0.05) (layer "F.Cu") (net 3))
 (segment (start 166.8 89.1) (end 153.3 89.1) (width 0.05) (layer "F.Cu") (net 3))
 (segment (start 171.8 98.6) (end 171.8 94.1) (width 0.05) (layer "F.Cu") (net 3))
 (segment (start 171.8 94.1) (end 166.8 89.1) (width 0.05) (layer "F.Cu") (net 3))
 (via (at 126.05 83.45) (size 0.6) (drill 0.3) (layers "F.Cu" "B.Cu") (free yes) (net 3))
 (segment (start 143.1 100.5) (end 145.6 100.5) (width 0.381) (layer "B.Cu") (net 3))
 (segment (start 126.05 83.45) (end 143.1 100.5) (width 0.381) (layer "B.Cu") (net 3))
 (segment (start 126.05 85.85) (end 126.05 88.04625) (width 0.381) (layer "F.Cu") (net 10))
 (segment (start 128.05 81.85) (end 128.05 83.85) (width 0.381) (layer "F.Cu") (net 10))
 (segment (start 128.05 83.85) (end 126.05 85.85) (width 0.381) (layer "F.Cu") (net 10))
 (segment (start 128.05 81.85) (end 130.55 81.85) (width 0.508) (layer "F.Cu") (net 10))
 (segment (start 120.3 77.6) (end 136.8 77.6) (width 0.05) (layer "F.Cu") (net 5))
 (segment (start 118.55 94.85) (end 114.275 94.85) (width 0.762) (layer "F.Cu") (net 5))
 (segment (start 119.3 94.1) (end 119.3 78.6) (width 0.05) (layer "F.Cu") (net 5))
 (segment (start 142.3 83.1) (end 146.95 83.1) (width 0.05) (layer "F.Cu") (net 5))
 (segment (start 118.55 94.85) (end 119.3 94.1) (width 0.05) (layer "F.Cu") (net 5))
 (segment (start 146.95 83.1) (end 148.6 81.45) (width 0.05) (layer "F.Cu") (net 5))
 (segment (start 136.8 77.6) (end 142.3 83.1) (width 0.05) (layer "F.Cu") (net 5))
 (segment (start 119.3 78.6) (end 120.3 77.6) (width 0.05) (layer "F.Cu") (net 5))
 (segment (start 173.05 99.35) (end 172.3 98.6) (width 0.05) (layer "F.Cu") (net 2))
 (segment (start 175.05 99.35) (end 179.445 94.955) (width 0.762) (layer "F.Cu") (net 2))
 (segment (start 167.3 88.6) (end 154.8 88.6) (width 0.05) (layer "F.Cu") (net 2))
 (segment (start 173.05 99.35) (end 175.05 99.35) (width 0.762) (layer "F.Cu") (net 2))
 (segment (start 152.35 86.15) (end 152.35 81.45) (width 0.05) (layer "F.Cu") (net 2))
 (segment (start 172.3 93.6) (end 167.3 88.6) (width 0.05) (layer "F.Cu") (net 2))
 (segment (start 179.445 94.955) (end 180.575 94.955) (width 0.762) (layer "F.Cu") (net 2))
 (segment (start 172.3 98.6) (end 172.3 93.6) (width 0.05) (layer "F.Cu") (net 2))
 (segment (start 154.8 88.6) (end 152.35 86.15) (width 0.05) (layer "F.Cu") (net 2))
 (segment (start 148.8 84.1) (end 149.85 83.05) (width 0.05) (layer "F.Cu") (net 4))
 (segment (start 120.55 94.85) (end 120.55 102.35) (width 0.762) (layer "F.Cu") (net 4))
 (segment (start 119.8 79.1) (end 120.8 78.1) (width 0.05) (layer "F.Cu") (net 4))
 (segment (start 142.3 84.1) (end 148.8 84.1) (width 0.05) (layer "F.Cu") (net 4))
 (segment (start 120.8 78.1) (end 136.3 78.1) (width 0.05) (layer "F.Cu") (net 4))
 (segment (start 149.85 83.05) (end 149.85 81.45) (width 0.05) (layer "F.Cu") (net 4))
 (segment (start 119.8 94.1) (end 119.8 79.1) (width 0.05) (layer "F.Cu") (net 4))
 (segment (start 120.55 102.35) (end 125.55 107.35) (width 0.762) (layer "F.Cu") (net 4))
 (segment (start 120.55 94.85) (end 119.8 94.1) (width 0.05) (layer "F.Cu") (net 4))
 (segment (start 136.3 78.1) (end 142.3 84.1) (width 0.05) (layer "F.Cu") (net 4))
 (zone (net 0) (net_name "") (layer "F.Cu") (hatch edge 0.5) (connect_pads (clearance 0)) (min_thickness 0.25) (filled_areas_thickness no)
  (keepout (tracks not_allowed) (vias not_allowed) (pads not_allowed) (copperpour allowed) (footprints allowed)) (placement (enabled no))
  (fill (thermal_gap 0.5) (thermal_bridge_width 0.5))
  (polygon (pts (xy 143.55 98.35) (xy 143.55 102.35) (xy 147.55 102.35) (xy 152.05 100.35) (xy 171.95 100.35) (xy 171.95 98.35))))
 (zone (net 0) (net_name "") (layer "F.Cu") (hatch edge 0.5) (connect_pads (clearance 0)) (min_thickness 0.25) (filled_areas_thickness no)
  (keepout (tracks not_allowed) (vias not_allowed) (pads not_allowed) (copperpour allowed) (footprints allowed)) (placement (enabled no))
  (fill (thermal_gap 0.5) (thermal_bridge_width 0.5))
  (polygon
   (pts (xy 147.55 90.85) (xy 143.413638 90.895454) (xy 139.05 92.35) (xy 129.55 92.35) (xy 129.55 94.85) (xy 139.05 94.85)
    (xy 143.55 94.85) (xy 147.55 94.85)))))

